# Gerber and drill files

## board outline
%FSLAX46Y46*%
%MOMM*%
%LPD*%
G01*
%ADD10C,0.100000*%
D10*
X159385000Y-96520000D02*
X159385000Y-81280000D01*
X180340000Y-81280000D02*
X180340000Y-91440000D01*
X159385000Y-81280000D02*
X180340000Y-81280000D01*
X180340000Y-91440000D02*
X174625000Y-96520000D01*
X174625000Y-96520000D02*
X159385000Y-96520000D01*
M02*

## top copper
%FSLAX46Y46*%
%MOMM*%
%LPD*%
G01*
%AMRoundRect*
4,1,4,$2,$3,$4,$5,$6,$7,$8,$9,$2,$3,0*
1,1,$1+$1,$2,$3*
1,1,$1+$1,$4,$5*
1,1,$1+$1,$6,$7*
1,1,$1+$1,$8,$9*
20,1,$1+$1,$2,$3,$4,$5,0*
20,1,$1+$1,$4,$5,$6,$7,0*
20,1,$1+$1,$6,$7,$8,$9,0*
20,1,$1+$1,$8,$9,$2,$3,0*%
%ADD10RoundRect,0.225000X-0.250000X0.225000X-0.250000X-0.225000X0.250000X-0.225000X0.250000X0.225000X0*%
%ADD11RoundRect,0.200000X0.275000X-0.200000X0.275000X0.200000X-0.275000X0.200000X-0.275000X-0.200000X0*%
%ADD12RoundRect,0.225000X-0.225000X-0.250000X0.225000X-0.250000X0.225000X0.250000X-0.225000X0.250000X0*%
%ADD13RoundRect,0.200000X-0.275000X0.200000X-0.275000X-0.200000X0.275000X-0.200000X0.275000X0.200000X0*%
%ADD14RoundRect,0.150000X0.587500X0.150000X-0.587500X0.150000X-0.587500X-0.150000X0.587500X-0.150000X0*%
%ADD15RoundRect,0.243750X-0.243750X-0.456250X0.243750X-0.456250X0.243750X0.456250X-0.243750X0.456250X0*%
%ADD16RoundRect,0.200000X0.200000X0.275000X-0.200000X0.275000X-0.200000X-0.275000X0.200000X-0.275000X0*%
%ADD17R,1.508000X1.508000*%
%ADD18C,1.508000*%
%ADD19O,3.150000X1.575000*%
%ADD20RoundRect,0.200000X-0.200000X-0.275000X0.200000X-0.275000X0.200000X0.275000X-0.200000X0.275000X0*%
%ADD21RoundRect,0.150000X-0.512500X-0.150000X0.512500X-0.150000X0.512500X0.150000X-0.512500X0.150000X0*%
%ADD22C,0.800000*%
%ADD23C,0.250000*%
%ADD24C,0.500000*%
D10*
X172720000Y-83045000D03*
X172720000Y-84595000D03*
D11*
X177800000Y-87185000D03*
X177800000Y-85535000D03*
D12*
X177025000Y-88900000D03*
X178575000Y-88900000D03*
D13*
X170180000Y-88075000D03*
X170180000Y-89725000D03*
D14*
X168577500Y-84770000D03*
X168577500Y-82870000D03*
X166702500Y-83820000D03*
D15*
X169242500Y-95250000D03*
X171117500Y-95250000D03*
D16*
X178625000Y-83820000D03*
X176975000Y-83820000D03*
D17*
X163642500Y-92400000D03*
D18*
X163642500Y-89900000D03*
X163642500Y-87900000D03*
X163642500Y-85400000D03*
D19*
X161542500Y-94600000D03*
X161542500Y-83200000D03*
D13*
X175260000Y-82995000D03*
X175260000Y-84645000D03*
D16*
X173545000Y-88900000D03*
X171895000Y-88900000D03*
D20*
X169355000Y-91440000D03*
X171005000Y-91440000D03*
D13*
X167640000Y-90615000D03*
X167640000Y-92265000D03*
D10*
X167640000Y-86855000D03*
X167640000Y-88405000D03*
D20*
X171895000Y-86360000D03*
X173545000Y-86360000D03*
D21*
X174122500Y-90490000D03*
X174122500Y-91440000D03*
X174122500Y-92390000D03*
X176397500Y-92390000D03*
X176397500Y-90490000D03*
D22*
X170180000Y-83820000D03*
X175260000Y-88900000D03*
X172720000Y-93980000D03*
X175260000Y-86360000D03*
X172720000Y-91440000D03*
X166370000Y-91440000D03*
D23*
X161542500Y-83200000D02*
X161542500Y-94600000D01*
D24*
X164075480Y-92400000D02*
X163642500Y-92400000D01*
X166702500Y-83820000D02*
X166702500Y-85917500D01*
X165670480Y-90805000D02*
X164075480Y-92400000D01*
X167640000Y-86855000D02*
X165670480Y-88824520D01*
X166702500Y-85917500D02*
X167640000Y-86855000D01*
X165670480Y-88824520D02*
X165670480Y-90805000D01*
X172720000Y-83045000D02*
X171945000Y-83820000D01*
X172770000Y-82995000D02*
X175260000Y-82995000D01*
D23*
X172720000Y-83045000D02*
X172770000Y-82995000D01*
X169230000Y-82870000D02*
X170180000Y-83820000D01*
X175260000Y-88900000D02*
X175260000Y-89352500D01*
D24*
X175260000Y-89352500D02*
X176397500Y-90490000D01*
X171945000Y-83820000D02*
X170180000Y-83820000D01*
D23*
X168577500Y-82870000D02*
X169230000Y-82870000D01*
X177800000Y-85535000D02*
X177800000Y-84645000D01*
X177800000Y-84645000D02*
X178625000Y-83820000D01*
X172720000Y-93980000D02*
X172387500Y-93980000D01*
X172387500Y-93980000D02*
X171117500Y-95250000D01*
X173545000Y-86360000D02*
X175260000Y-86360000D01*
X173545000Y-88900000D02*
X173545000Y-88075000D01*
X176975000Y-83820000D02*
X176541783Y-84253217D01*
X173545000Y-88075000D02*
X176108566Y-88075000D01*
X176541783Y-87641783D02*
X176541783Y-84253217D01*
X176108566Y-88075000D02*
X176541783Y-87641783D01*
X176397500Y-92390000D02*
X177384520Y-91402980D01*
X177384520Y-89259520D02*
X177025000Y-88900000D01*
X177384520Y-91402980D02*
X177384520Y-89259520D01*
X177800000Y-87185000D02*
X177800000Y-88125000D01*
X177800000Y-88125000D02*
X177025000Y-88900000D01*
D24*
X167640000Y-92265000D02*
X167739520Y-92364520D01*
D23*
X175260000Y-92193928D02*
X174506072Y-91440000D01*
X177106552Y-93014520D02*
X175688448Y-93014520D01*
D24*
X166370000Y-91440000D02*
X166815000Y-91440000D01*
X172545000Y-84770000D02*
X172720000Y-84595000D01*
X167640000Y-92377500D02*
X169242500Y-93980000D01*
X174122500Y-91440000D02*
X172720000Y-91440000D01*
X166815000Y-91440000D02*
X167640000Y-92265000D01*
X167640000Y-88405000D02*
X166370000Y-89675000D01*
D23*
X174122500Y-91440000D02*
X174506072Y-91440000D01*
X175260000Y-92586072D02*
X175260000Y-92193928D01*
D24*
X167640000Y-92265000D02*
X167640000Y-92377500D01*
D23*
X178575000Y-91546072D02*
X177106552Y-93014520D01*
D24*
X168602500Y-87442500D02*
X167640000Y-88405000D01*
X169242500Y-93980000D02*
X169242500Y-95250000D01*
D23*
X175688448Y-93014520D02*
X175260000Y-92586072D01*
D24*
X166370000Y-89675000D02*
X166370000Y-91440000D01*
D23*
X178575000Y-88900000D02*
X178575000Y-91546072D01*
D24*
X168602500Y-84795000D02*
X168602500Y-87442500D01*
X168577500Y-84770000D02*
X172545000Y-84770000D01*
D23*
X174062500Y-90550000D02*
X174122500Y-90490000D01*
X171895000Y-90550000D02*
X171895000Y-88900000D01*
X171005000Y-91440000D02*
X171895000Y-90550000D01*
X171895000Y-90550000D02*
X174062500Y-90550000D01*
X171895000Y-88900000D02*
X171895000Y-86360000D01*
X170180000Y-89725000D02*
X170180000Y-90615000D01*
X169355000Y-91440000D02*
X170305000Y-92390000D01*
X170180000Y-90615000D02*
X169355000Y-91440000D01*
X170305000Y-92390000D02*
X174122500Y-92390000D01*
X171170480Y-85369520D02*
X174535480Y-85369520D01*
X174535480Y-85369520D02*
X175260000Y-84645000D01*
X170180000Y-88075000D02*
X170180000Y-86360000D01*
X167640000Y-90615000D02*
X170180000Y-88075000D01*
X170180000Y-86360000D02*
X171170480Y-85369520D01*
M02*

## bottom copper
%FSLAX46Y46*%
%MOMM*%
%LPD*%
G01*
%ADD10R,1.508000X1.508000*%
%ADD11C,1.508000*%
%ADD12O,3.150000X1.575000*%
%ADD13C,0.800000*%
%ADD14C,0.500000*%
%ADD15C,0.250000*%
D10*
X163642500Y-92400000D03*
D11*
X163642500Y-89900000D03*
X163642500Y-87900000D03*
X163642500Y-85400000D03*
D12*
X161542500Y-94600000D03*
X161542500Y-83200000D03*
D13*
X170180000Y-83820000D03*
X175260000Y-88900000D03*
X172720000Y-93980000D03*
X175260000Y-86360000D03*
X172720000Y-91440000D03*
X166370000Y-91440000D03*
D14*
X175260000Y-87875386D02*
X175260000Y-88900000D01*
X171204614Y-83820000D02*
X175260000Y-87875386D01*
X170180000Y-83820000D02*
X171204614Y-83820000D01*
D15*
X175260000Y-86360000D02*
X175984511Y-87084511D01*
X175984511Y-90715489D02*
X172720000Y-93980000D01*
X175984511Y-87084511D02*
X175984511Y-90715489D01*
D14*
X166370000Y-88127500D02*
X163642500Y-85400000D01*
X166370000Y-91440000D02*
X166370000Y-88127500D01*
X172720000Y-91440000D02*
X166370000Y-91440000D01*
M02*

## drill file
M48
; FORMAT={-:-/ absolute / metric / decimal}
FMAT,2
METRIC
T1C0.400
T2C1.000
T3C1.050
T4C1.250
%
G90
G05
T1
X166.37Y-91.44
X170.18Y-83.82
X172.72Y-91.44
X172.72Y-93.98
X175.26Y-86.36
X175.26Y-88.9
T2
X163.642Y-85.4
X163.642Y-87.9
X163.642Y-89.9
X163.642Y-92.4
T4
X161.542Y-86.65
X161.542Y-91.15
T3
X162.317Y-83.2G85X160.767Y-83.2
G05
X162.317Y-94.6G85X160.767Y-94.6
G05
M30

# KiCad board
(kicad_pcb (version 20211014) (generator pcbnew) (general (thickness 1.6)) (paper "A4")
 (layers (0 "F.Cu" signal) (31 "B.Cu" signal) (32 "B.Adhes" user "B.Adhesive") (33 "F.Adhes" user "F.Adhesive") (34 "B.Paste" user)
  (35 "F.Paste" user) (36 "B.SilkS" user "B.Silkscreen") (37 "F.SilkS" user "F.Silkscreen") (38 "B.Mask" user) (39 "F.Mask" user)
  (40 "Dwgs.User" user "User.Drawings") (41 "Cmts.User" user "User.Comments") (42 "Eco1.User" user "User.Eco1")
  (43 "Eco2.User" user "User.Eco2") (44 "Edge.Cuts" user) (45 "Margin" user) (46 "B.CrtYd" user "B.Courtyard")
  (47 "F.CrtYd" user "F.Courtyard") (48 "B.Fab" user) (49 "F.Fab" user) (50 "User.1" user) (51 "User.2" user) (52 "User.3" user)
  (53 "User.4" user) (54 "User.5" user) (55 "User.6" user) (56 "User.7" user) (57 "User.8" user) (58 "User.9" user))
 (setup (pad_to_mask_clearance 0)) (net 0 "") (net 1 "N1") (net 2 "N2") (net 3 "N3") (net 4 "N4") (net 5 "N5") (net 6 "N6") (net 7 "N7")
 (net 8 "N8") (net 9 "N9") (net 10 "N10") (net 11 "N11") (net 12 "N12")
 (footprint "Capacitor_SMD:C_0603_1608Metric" (layer "F.Cu") (at 172.72 83.82 -90)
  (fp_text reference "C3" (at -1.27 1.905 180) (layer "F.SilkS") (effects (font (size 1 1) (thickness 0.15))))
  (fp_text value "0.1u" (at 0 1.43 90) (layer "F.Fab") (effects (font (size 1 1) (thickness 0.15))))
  (pad "1" smd roundrect (at -0.775 0 270) (size 0.9 0.95) (layers "F.Cu" "F.Paste" "F.Mask") (roundrect_rratio 0.25) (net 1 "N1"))
  (pad "2" smd roundrect (at 0.775 0 270) (size 0.9 0.95) (layers "F.Cu" "F.Paste" "F.Mask") (roundrect_rratio 0.25) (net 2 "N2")))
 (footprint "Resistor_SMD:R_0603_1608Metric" (layer "F.Cu") (at 177.8 86.36 90)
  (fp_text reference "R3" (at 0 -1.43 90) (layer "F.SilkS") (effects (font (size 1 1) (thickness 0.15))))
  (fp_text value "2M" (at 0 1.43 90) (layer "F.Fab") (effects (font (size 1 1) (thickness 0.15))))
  (pad "1" smd roundrect (at -0.825 0 90) (size 0.8 0.95) (layers "F.Cu" "F.Paste" "F.Mask") (roundrect_rratio 0.25) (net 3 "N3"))
  (pad "2" smd roundrect (at 0.825 0 90) (size 0.8 0.95) (layers "F.Cu" "F.Paste" "F.Mask") (roundrect_rratio 0.25) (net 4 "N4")))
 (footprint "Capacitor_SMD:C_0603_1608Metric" (layer "F.Cu") (at 177.8 88.9)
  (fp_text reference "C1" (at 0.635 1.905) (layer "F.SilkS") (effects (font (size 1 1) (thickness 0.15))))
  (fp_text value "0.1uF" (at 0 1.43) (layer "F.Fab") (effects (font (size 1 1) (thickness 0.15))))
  (pad "1" smd roundrect (at -0.775 0) (size 0.9 0.95) (layers "F.Cu" "F.Paste" "F.Mask") (roundrect_rratio 0.25) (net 3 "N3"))
  (pad "2" smd roundrect (at 0.775 0) (size 0.9 0.95) (layers "F.Cu" "F.Paste" "F.Mask") (roundrect_rratio 0.25) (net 2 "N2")))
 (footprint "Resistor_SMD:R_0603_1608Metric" (layer "F.Cu") (at 170.18 88.9 -90)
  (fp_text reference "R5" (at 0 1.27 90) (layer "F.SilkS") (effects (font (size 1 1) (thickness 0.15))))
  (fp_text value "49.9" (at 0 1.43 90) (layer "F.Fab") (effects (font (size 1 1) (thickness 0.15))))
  (pad "1" smd roundrect (at -0.825 0 270) (size 0.8 0.95) (layers "F.Cu" "F.Paste" "F.Mask") (roundrect_rratio 0.25) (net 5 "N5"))
  (pad "2" smd roundrect (at 0.825 0 270) (size 0.8 0.95) (layers "F.Cu" "F.Paste" "F.Mask") (roundrect_rratio 0.25) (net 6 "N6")))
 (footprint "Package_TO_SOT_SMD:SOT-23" (layer "F.Cu") (at 167.64 83.82 180)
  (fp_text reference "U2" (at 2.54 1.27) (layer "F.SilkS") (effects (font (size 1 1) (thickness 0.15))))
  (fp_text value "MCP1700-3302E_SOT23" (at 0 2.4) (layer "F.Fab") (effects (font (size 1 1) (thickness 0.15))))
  (pad "1" smd roundrect (at -0.9375 -0.95 180) (size 1.475 0.6) (layers "F.Cu" "F.Paste" "F.Mask") (roundrect_rratio 0.25) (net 2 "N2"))
  (pad "2" smd roundrect (at -0.9375 0.95 180) (size 1.475 0.6) (layers "F.Cu" "F.Paste" "F.Mask") (roundrect_rratio 0.25) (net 1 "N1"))
  (pad "3" smd roundrect (at 0.9375 0 180) (size 1.475 0.6) (layers "F.Cu" "F.Paste" "F.Mask") (roundrect_rratio 0.25) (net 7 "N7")))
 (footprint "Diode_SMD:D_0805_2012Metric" (layer "F.Cu") (at 170.18 95.25)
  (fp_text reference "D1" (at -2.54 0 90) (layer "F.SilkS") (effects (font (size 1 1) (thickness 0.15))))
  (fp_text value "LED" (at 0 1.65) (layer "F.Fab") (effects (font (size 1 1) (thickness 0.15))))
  (pad "1" smd roundrect (at -0.9375 0) (size 0.975 1.4) (layers "F.Cu" "F.Paste" "F.Mask") (roundrect_rratio 0.25) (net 2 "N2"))
  (pad "2" smd roundrect (at 0.9375 0) (size 0.975 1.4) (layers "F.Cu" "F.Paste" "F.Mask") (roundrect_rratio 0.25) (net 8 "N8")))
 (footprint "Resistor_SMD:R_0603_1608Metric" (layer "F.Cu") (at 177.8 83.82 180)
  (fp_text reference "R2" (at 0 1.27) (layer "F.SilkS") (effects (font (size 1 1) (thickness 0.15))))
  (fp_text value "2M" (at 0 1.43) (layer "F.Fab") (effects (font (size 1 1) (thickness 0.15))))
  (pad "1" smd roundrect (at -0.825 0 180) (size 0.8 0.95) (layers "F.Cu" "F.Paste" "F.Mask") (roundrect_rratio 0.25) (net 4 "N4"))
  (pad "2" smd roundrect (at 0.825 0 180) (size 0.8 0.95) (layers "F.Cu" "F.Paste" "F.Mask") (roundrect_rratio 0.25) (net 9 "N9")))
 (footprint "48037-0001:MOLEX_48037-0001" (layer "F.Cu") (at 161.5425 88.9 -90)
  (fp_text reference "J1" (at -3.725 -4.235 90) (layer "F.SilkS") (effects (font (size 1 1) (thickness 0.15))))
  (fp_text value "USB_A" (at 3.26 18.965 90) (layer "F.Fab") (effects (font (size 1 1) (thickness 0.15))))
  (pad "" np_thru_hole circle (at -2.25 0 270) (size 1.25 1.25) (drill 1.25) (layers *.Cu *.Mask))
  (pad "" np_thru_hole circle (at 2.25 0 270) (size 1.25 1.25) (drill 1.25) (layers *.Cu *.Mask))
  (pad "1" thru_hole rect (at 3.5 -2.1 270) (size 1.508 1.508) (drill 1) (layers *.Cu *.Mask) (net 7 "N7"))
  (pad "2" thru_hole circle (at 1 -2.1 270) (size 1.508 1.508) (drill 1) (layers *.Cu *.Mask) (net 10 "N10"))
  (pad "3" thru_hole circle (at -1 -2.1 270) (size 1.508 1.508) (drill 1) (layers *.Cu *.Mask) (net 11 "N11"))
  (pad "4" thru_hole circle (at -3.5 -2.1 270) (size 1.508 1.508) (drill 1) (layers *.Cu *.Mask) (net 2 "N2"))
  (pad "S1" thru_hole oval (at 5.7 0 270) (size 1.575 3.15) (drill oval 1.05 2.6) (layers *.Cu *.Mask))
  (pad "S2" thru_hole oval (at -5.7 0 270) (size 1.575 3.15) (drill oval 1.05 2.6) (layers *.Cu *.Mask)))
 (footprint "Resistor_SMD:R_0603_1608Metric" (layer "F.Cu") (at 175.26 83.82 -90)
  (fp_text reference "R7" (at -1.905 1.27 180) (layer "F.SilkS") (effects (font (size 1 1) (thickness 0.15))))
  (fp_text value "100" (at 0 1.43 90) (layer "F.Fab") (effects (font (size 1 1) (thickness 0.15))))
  (pad "1" smd roundrect (at -0.825 0 270) (size 0.8 0.95) (layers "F.Cu" "F.Paste" "F.Mask") (roundrect_rratio 0.25) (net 1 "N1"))
  (pad "2" smd roundrect (at 0.825 0 270) (size 0.8 0.95) (layers "F.Cu" "F.Paste" "F.Mask") (roundrect_rratio 0.25) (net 5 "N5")))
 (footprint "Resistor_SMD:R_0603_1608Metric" (layer "F.Cu") (at 172.72 88.9 180)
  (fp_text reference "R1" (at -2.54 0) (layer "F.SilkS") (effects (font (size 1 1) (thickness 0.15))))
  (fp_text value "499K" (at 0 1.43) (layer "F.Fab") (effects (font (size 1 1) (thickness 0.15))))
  (pad "1" smd roundrect (at -0.825 0 180) (size 0.8 0.95) (layers "F.Cu" "F.Paste" "F.Mask") (roundrect_rratio 0.25) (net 9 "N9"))
  (pad "2" smd roundrect (at 0.825 0 180) (size 0.8 0.95) (layers "F.Cu" "F.Paste" "F.Mask") (roundrect_rratio 0.25) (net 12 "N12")))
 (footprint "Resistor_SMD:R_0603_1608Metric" (layer "F.Cu") (at 170.18 91.44)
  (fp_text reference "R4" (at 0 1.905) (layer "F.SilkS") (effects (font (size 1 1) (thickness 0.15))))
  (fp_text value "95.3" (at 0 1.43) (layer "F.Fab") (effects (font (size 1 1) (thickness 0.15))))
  (pad "1" smd roundrect (at -0.825 0) (size 0.8 0.95) (layers "F.Cu" "F.Paste" "F.Mask") (roundrect_rratio 0.25) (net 6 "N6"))
  (pad "2" smd roundrect (at 0.825 0) (size 0.8 0.95) (layers "F.Cu" "F.Paste" "F.Mask") (roundrect_rratio 0.25) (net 12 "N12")))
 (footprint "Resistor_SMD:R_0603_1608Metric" (layer "F.Cu") (at 167.64 91.44 -90)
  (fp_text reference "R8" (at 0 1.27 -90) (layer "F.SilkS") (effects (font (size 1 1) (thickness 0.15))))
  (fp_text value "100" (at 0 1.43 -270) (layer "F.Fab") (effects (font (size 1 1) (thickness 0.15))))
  (pad "1" smd roundrect (at -0.825 0 270) (size 0.8 0.95) (layers "F.Cu" "F.Paste" "F.Mask") (roundrect_rratio 0.25) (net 5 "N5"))
  (pad "2" smd roundrect (at 0.825 0 270) (size 0.8 0.95) (layers "F.Cu" "F.Paste" "F.Mask") (roundrect_rratio 0.25) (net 2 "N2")))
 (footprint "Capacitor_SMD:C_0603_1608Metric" (layer "F.Cu") (at 167.64 87.63 -90)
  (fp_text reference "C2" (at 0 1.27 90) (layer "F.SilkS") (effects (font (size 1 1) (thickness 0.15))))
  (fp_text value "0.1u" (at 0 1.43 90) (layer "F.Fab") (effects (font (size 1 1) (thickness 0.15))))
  (pad "1" smd roundrect (at -0.775 0 270) (size 0.9 0.95) (layers "F.Cu" "F.Paste" "F.Mask") (roundrect_rratio 0.25) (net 7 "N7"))
  (pad "2" smd roundrect (at 0.775 0 270) (size 0.9 0.95) (layers "F.Cu" "F.Paste" "F.Mask") (roundrect_rratio 0.25) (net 2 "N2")))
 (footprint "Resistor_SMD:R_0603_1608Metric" (layer "F.Cu") (at 172.72 86.36)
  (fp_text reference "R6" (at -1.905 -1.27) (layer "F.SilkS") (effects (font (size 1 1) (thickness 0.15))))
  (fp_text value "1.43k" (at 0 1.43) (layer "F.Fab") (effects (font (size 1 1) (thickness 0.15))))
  (pad "1" smd roundrect (at -0.825 0) (size 0.8 0.95) (layers "F.Cu" "F.Paste" "F.Mask") (roundrect_rratio 0.25) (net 12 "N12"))
  (pad "2" smd roundrect (at 0.825 0) (size 0.8 0.95) (layers "F.Cu" "F.Paste" "F.Mask") (roundrect_rratio 0.25) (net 8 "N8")))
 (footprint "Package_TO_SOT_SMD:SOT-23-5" (layer "F.Cu") (at 175.26 91.44)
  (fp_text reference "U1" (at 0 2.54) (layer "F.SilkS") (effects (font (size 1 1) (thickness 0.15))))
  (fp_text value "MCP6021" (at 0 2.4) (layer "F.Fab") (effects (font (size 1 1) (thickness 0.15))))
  (pad "1" smd roundrect (at -1.1375 -0.95) (size 1.325 0.6) (layers "F.Cu" "F.Paste" "F.Mask") (roundrect_rratio 0.25) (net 12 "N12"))
  (pad "2" smd roundrect (at -1.1375 0) (size 1.325 0.6) (layers "F.Cu" "F.Paste" "F.Mask") (roundrect_rratio 0.25) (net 2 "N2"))
  (pad "3" smd roundrect (at -1.1375 0.95) (size 1.325 0.6) (layers "F.Cu" "F.Paste" "F.Mask") (roundrect_rratio 0.25) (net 6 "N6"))
  (pad "4" smd roundrect (at 1.1375 0.95) (size 1.325 0.6) (layers "F.Cu" "F.Paste" "F.Mask") (roundrect_rratio 0.25) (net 3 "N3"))
  (pad "5" smd roundrect (at 1.1375 -0.95) (size 1.325 0.6) (layers "F.Cu" "F.Paste" "F.Mask") (roundrect_rratio 0.25) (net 1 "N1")))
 (gr_line (start 159.385 96.52) (end 159.385 81.28) (layer "Edge.Cuts") (width 0.1))
 (gr_line (start 180.34 81.28) (end 180.34 91.44) (layer "Edge.Cuts") (width 0.1))
 (gr_line (start 159.385 81.28) (end 180.34 81.28) (layer "Edge.Cuts") (width 0.1))
 (gr_line (start 180.34 91.44) (end 174.625 96.52) (layer "Edge.Cuts") (width 0.1))
 (gr_line (start 174.625 96.52) (end 159.385 96.52) (layer "Edge.Cuts") (width 0.1))
 (segment (start 161.5425 83.2) (end 161.5425 94.6) (width 0.25) (layer "F.Cu") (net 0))
 (segment (start 164.07548 92.4) (end 163.6425 92.4) (width 0.5) (layer "F.Cu") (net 7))
 (segment (start 166.7025 83.82) (end 166.7025 85.9175) (width 0.5) (layer "F.Cu") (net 7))
 (segment (start 165.67048 90.805) (end 164.07548 92.4) (width 0.5) (layer "F.Cu") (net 7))
 (segment (start 167.64 86.855) (end 165.67048 88.82452) (width 0.5) (layer "F.Cu") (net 7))
 (segment (start 166.7025 85.9175) (end 167.64 86.855) (width 0.5) (layer "F.Cu") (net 7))
 (segment (start 165.67048 88.82452) (end 165.67048 90.805) (width 0.5) (layer "F.Cu") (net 7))
 (segment (start 172.72 83.045) (end 171.945 83.82) (width 0.5) (layer "F.Cu") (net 1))
 (segment (start 172.77 82.995) (end 175.26 82.995) (width 0.5) (layer "F.Cu") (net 1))
 (segment (start 172.72 83.045) (end 172.77 82.995) (width 0.25) (layer "F.Cu") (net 1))
 (segment (start 169.23 82.87) (end 170.18 83.82) (width 0.25) (layer "F.Cu") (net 1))
 (segment (start 175.26 88.9) (end 175.26 89.3525) (width 0.25) (layer "F.Cu") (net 1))
 (segment (start 175.26 89.3525) (end 176.3975 90.49) (width 0.5) (layer "F.Cu") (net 1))
 (segment (start 171.945 83.82) (end 170.18 83.82) (width 0.5) (layer "F.Cu") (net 1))
 (segment (start 168.5775 82.87) (end 169.23 82.87) (width 0.25) (layer "F.Cu") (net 1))
 (via (at 170.18 83.82) (size 0.8) (drill 0.4) (layers "F.Cu" "B.Cu") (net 1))
 (via (at 175.26 88.9) (size 0.8) (drill 0.4) (layers "F.Cu" "B.Cu") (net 1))
 (segment (start 175.26 87.875386) (end 175.26 88.9) (width 0.5) (layer "B.Cu") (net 1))
 (segment (start 171.204614 83.82) (end 175.26 87.875386) (width 0.5) (layer "B.Cu") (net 1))
 (segment (start 170.18 83.82) (end 171.204614 83.82) (width 0.5) (layer "B.Cu") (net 1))
 (segment (start 177.8 85.535) (end 177.8 84.645) (width 0.25) (layer "F.Cu") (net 4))
 (segment (start 177.8 84.645) (end 178.625 83.82) (width 0.25) (layer "F.Cu") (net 4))
 (segment (start 172.72 93.98) (end 172.3875 93.98) (width 0.25) (layer "F.Cu") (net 8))
 (segment (start 172.3875 93.98) (end 171.1175 95.25) (width 0.25) (layer "F.Cu") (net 8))
 (segment (start 173.545 86.36) (end 175.26 86.36) (width 0.25) (layer "F.Cu") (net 8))
 (via (at 172.72 93.98) (size 0.8) (drill 0.4) (layers "F.Cu" "B.Cu") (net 8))
 (via (at 175.26 86.36) (size 0.8) (drill 0.4) (layers "F.Cu" "B.Cu") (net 8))
 (segment (start 175.26 86.36) (end 175.984511 87.084511) (width 0.25) (layer "B.Cu") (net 8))
 (segment (start 175.984511 90.715489) (end 172.72 93.98) (width 0.25) (layer "B.Cu") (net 8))
 (segment (start 175.984511 87.084511) (end 175.984511 90.715489) (width 0.25) (layer "B.Cu") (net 8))
 (segment (start 173.545 88.9) (end 173.545 88.075) (width 0.25) (layer "F.Cu") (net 9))
 (segment (start 176.975 83.82) (end 176.541783 84.253217) (width 0.25) (layer "F.Cu") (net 9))
 (segment (start 173.545 88.075) (end 176.108566 88.075) (width 0.25) (layer "F.Cu") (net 9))
 (segment (start 176.541783 87.641783) (end 176.541783 84.253217) (width 0.25) (layer "F.Cu") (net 9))
 (segment (start 176.108566 88.075) (end 176.541783 87.641783) (width 0.25) (layer "F.Cu") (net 9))
 (segment (start 176.3975 92.39) (end 177.38452 91.40298) (width 0.25) (layer "F.Cu") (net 3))
 (segment (start 177.38452 89.25952) (end 177.025 88.9) (width 0.25) (layer "F.Cu") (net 3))
 (segment (start 177.38452 91.40298) (end 177.38452 89.25952) (width 0.25) (layer "F.Cu") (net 3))
 (segment (start 177.8 87.185) (end 177.8 88.125) (width 0.25) (layer "F.Cu") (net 3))
 (segment (start 177.8 88.125) (end 177.025 88.9) (width 0.25) (layer "F.Cu") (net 3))
 (segment (start 167.64 92.265) (end 167.73952 92.36452) (width 0.5) (layer "F.Cu") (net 2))
 (segment (start 175.26 92.193928) (end 174.506072 91.44) (width 0.25) (layer "F.Cu") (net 2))
 (segment (start 177.106552 93.01452) (end 175.688448 93.01452) (width 0.25) (layer "F.Cu") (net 2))
 (segment (start 166.37 91.44) (end 166.815 91.44) (width 0.5) (layer "F.Cu") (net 2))
 (segment (start 172.545 84.77) (end 172.72 84.595) (width 0.5) (layer "F.Cu") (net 2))
 (segment (start 167.64 92.3775) (end 169.2425 93.98) (width 0.5) (layer "F.Cu") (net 2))
 (segment (start 174.1225 91.44) (end 172.72 91.44) (width 0.5) (layer "F.Cu") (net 2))
 (segment (start 166.815 91.44) (end 167.64 92.265) (width 0.5) (layer "F.Cu") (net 2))
 (segment (start 167.64 88.405) (end 166.37 89.675) (width 0.5) (layer "F.Cu") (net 2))
 (segment (start 174.1225 91.44) (end 174.506072 91.44) (width 0.25) (layer "F.Cu") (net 2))
 (segment (start 175.26 92.586072) (end 175.26 92.193928) (width 0.25) (layer "F.Cu") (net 2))
 (segment (start 167.64 92.265) (end 167.64 92.3775) (width 0.5) (layer "F.Cu") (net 2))
 (segment (start 178.575 91.546072) (end 177.106552 93.01452) (width 0.25) (layer "F.Cu") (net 2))
 (segment (start 168.6025 87.4425) (end 167.64 88.405) (width 0.5) (layer "F.Cu") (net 2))
 (segment (start 169.2425 93.98) (end 169.2425 95.25) (width 0.5) (layer "F.Cu") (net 2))
 (segment (start 175.688448 93.01452) (end 175.26 92.586072) (width 0.25) (layer "F.Cu") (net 2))
 (segment (start 166.37 89.675) (end 166.37 91.44) (width 0.5) (layer "F.Cu") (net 2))
 (segment (start 178.575 88.9) (end 178.575 91.546072) (width 0.25) (layer "F.Cu") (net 2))
 (segment (start 168.6025 84.795) (end 168.6025 87.4425) (width 0.5) (layer "F.Cu") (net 2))
 (segment (start 168.5775 84.77) (end 172.545 84.77) (width 0.5) (layer "F.Cu") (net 2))
 (via (at 172.72 91.44) (size 0.8) (drill 0.4) (layers "F.Cu" "B.Cu") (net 2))
 (via (at 166.37 91.44) (size 0.8) (drill 0.4) (layers "F.Cu" "B.Cu") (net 2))
 (segment (start 166.37 88.1275) (end 163.6425 85.4) (width 0.5) (layer "B.Cu") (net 2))
 (segment (start 166.37 91.44) (end 166.37 88.1275) (width 0.5) (layer "B.Cu") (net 2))
 (segment (start 172.72 91.44) (end 166.37 91.44) (width 0.5) (layer "B.Cu") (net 2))
 (segment (start 174.0625 90.55) (end 174.1225 90.49) (width 0.25) (layer "F.Cu") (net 12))
 (segment (start 171.895 90.55) (end 171.895 88.9) (width 0.25) (layer "F.Cu") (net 12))
 (segment (start 171.005 91.44) (end 171.895 90.55) (width 0.25) (layer "F.Cu") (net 12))
 (segment (start 171.895 90.55) (end 174.0625 90.55) (width 0.25) (layer "F.Cu") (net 12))
 (segment (start 171.895 88.9) (end 171.895 86.36) (width 0.25) (layer "F.Cu") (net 12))
 (segment (start 170.18 89.725) (end 170.18 90.615) (width 0.25) (layer "F.Cu") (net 6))
 (segment (start 169.355 91.44) (end 170.305 92.39) (width 0.25) (layer "F.Cu") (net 6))
 (segment (start 170.18 90.615) (end 169.355 91.44) (width 0.25) (layer "F.Cu") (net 6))
 (segment (start 170.305 92.39) (end 174.1225 92.39) (width 0.25) (layer "F.Cu") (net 6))
 (segment (start 171.17048 85.36952) (end 174.53548 85.36952) (width 0.25) (layer "F.Cu") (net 5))
 (segment (start 174.53548 85.36952) (end 175.26 84.645) (width 0.25) (layer "F.Cu") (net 5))
 (segment (start 170.18 88.075) (end 170.18 86.36) (width 0.25) (layer "F.Cu") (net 5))
 (segment (start 167.64 90.615) (end 170.18 88.075) (width 0.25) (layer "F.Cu") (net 5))
 (segment (start 170.18 86.36) (end 171.17048 85.36952) (width 0.25) (layer "F.Cu") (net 5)))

